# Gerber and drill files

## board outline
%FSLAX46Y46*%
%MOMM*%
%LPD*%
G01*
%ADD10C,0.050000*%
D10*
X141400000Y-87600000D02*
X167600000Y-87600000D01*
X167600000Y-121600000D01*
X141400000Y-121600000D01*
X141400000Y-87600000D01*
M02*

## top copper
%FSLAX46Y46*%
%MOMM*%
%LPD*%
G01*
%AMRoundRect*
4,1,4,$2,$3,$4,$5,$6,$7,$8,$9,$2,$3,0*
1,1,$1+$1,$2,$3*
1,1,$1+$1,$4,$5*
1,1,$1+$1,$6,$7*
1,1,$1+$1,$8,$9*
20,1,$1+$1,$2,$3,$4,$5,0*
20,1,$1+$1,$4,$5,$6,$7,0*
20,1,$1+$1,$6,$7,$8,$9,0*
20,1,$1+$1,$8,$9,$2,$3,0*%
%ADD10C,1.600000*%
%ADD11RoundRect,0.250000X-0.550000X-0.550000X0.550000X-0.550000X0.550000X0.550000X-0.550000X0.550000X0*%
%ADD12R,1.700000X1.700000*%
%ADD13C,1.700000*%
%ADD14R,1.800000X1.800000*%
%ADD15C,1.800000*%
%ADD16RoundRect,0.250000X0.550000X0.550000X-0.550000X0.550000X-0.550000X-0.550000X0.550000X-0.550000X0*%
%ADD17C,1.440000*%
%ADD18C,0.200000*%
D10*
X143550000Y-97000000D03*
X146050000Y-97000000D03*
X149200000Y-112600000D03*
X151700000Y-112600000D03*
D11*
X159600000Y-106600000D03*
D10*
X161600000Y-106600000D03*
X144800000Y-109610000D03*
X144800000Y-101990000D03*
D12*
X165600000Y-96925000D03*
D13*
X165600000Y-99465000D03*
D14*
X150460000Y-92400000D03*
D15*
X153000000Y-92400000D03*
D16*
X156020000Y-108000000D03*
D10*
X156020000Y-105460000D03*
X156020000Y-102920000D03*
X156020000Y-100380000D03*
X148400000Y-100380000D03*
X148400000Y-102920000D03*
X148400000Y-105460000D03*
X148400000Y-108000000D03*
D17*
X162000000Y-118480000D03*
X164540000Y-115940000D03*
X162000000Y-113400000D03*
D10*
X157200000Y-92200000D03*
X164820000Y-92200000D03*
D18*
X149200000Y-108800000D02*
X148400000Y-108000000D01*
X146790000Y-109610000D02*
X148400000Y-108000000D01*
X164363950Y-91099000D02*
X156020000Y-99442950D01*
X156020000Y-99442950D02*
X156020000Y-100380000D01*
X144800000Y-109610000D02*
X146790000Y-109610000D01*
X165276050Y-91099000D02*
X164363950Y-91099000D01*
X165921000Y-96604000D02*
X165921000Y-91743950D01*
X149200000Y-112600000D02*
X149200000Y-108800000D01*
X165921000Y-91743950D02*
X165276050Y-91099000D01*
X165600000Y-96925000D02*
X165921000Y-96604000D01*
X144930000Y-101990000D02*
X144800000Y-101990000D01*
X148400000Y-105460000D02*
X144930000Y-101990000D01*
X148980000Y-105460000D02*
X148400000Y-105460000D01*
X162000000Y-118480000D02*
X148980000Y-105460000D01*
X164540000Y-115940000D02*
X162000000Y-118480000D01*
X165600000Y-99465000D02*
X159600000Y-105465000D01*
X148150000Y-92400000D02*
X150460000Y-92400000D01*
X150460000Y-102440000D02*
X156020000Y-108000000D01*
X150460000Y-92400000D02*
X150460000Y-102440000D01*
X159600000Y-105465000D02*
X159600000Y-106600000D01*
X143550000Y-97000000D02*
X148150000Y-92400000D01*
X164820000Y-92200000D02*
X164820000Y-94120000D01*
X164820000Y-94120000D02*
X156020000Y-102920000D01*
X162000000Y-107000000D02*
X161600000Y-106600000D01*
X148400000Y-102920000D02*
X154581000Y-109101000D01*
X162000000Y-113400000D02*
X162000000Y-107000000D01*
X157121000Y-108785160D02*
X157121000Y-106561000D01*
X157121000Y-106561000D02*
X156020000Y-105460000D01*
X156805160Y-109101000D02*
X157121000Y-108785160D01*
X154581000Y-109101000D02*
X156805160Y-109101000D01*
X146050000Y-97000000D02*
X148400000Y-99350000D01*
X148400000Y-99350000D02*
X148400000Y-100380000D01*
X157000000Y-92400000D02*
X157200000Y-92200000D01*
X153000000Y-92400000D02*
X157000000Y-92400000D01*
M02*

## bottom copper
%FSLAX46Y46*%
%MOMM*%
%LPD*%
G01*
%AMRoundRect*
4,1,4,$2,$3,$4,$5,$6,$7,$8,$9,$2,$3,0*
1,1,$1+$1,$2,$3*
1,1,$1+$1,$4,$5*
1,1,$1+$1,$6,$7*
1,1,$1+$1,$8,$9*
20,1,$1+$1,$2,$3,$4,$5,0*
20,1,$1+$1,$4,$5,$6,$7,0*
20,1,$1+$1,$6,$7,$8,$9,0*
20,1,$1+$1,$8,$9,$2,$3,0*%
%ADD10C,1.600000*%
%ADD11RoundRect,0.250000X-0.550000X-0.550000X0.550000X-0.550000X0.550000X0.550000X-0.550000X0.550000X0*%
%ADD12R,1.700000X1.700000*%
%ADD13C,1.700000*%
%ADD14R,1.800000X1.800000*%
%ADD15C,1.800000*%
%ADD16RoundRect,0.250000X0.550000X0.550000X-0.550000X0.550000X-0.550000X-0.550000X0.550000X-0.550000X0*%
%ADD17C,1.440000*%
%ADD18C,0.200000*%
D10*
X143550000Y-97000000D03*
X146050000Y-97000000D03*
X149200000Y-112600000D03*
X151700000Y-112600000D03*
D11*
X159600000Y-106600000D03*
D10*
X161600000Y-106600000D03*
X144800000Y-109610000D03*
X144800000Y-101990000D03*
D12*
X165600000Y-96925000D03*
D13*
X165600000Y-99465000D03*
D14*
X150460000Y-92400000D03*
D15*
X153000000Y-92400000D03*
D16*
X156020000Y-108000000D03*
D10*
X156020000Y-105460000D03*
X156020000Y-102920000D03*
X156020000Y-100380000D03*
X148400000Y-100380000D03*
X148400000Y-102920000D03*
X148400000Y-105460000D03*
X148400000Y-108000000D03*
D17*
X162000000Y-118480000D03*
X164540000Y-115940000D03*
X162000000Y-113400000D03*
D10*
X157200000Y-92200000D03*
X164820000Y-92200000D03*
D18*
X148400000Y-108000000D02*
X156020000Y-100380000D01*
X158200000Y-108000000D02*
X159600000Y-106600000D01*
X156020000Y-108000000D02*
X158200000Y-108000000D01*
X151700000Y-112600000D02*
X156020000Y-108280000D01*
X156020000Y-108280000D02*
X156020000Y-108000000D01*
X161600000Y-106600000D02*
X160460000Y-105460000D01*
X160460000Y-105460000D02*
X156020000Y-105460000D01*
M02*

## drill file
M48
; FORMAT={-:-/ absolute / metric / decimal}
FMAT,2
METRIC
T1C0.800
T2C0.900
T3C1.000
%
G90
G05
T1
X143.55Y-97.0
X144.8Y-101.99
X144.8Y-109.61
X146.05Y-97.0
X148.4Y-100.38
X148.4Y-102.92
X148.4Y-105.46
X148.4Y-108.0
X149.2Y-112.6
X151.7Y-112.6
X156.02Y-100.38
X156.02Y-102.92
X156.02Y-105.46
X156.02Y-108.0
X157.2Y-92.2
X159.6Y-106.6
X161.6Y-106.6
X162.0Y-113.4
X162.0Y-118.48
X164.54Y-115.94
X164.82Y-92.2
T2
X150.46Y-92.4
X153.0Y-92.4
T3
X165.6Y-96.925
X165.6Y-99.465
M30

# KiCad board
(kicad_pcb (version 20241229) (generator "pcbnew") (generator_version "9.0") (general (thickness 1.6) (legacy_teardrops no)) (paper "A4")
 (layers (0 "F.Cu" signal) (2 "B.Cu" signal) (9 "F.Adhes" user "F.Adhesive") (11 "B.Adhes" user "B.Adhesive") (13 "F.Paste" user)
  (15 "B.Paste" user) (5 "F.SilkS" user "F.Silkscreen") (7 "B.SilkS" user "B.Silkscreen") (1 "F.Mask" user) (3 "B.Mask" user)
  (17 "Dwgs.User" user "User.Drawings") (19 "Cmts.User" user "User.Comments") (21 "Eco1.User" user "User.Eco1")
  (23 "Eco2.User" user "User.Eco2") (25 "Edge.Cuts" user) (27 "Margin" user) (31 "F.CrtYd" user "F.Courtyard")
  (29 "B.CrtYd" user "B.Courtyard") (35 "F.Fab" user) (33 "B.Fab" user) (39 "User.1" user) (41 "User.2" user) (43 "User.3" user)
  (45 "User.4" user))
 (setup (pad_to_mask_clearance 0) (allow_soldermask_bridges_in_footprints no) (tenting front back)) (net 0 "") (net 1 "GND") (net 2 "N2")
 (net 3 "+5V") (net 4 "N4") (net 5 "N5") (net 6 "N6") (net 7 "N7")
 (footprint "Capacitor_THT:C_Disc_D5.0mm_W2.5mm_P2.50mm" (layer "F.Cu") (at 143.55 97)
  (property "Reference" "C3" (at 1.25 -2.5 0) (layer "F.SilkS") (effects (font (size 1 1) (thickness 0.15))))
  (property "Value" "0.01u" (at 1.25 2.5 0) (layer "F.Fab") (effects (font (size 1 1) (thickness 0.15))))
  (pad "1" thru_hole circle (at 0 0) (size 1.6 1.6) (drill 0.8) (layers "*.Cu" "*.Mask") (remove_unused_layers no) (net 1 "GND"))
  (pad "2" thru_hole circle (at 2.5 0) (size 1.6 1.6) (drill 0.8) (layers "*.Cu" "*.Mask") (remove_unused_layers no) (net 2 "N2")))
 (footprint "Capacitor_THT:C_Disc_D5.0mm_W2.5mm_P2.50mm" (layer "F.Cu") (at 149.2 112.6)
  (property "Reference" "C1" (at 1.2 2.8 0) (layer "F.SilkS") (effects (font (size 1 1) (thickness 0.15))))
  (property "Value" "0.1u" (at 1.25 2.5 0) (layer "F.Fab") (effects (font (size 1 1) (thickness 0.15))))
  (pad "1" thru_hole circle (at 0 0) (size 1.6 1.6) (drill 0.8) (layers "*.Cu" "*.Mask") (remove_unused_layers no) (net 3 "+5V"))
  (pad "2" thru_hole circle (at 2.5 0) (size 1.6 1.6) (drill 0.8) (layers "*.Cu" "*.Mask") (remove_unused_layers no) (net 1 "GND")))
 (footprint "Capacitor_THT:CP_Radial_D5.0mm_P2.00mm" (layer "F.Cu") (at 159.6 106.6)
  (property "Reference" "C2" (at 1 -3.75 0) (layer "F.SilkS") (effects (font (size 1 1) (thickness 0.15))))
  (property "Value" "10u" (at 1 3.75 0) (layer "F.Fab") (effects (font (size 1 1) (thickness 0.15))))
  (pad "1" thru_hole roundrect (at 0 0) (size 1.6 1.6) (drill 0.8) (layers "*.Cu" "*.Mask") (remove_unused_layers no)
   (roundrect_rratio 0.15625) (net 1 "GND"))
  (pad "2" thru_hole circle (at 2 0) (size 1.6 1.6) (drill 0.8) (layers "*.Cu" "*.Mask") (remove_unused_layers no) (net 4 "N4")))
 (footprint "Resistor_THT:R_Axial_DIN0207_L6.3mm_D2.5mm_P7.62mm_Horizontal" (layer "F.Cu") (at 144.8 109.61 90)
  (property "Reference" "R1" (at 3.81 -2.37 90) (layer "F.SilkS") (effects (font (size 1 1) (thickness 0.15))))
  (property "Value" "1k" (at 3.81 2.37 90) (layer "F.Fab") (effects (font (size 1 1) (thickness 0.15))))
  (pad "1" thru_hole circle (at 0 0 90) (size 1.6 1.6) (drill 0.8) (layers "*.Cu" "*.Mask") (remove_unused_layers no) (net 3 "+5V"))
  (pad "2" thru_hole circle (at 7.62 0 90) (size 1.6 1.6) (drill 0.8) (layers "*.Cu" "*.Mask") (remove_unused_layers no) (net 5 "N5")))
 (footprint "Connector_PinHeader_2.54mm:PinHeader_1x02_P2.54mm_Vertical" (layer "F.Cu") (at 165.6 96.925)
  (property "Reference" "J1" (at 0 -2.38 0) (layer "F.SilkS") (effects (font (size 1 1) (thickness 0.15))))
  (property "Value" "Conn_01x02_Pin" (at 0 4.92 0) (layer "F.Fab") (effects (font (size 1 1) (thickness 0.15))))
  (pad "1" thru_hole rect (at 0 0) (size 1.7 1.7) (drill 1) (layers "*.Cu" "*.Mask") (remove_unused_layers no) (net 3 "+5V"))
  (pad "2" thru_hole circle (at 0 2.54) (size 1.7 1.7) (drill 1) (layers "*.Cu" "*.Mask") (remove_unused_layers no) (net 1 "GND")))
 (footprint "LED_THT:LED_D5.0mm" (layer "F.Cu") (at 150.46 92.4)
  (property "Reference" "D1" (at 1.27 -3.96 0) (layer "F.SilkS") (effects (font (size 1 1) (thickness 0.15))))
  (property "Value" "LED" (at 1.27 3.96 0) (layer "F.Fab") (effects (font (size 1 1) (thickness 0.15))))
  (pad "1" thru_hole rect (at 0 0) (size 1.8 1.8) (drill 0.9) (layers "*.Cu" "*.Mask") (remove_unused_layers no) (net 1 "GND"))
  (pad "2" thru_hole circle (at 2.54 0) (size 1.8 1.8) (drill 0.9) (layers "*.Cu" "*.Mask") (remove_unused_layers no) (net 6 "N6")))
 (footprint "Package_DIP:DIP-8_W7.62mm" (layer "F.Cu") (at 156.02 108 180)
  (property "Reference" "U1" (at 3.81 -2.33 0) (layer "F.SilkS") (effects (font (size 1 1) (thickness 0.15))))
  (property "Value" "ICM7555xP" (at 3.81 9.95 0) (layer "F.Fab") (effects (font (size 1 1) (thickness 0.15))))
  (pad "1" thru_hole roundrect (at 0 0 180) (size 1.6 1.6) (drill 0.8) (layers "*.Cu" "*.Mask") (remove_unused_layers no)
   (roundrect_rratio 0.15625) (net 1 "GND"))
  (pad "2" thru_hole circle (at 0 2.54 180) (size 1.6 1.6) (drill 0.8) (layers "*.Cu" "*.Mask") (remove_unused_layers no) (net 4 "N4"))
  (pad "3" thru_hole circle (at 0 5.08 180) (size 1.6 1.6) (drill 0.8) (layers "*.Cu" "*.Mask") (remove_unused_layers no) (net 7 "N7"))
  (pad "4" thru_hole circle (at 0 7.62 180) (size 1.6 1.6) (drill 0.8) (layers "*.Cu" "*.Mask") (remove_unused_layers no) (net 3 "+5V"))
  (pad "5" thru_hole circle (at 7.62 7.62 180) (size 1.6 1.6) (drill 0.8) (layers "*.Cu" "*.Mask") (remove_unused_layers no) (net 2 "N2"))
  (pad "6" thru_hole circle (at 7.62 5.08 180) (size 1.6 1.6) (drill 0.8) (layers "*.Cu" "*.Mask") (remove_unused_layers no) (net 4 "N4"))
  (pad "7" thru_hole circle (at 7.62 2.54 180) (size 1.6 1.6) (drill 0.8) (layers "*.Cu" "*.Mask") (remove_unused_layers no) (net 5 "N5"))
  (pad "8" thru_hole circle (at 7.62 0 180) (size 1.6 1.6) (drill 0.8) (layers "*.Cu" "*.Mask") (remove_unused_layers no) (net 3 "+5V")))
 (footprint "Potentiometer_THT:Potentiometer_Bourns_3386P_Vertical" (layer "F.Cu") (at 162 118.48)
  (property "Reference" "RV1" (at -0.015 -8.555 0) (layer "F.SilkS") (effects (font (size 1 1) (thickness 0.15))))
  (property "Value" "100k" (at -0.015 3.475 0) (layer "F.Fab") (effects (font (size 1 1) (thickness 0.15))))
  (pad "1" thru_hole circle (at 0 0) (size 1.44 1.44) (drill 0.8) (layers "*.Cu" "*.Mask") (remove_unused_layers no) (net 5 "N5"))
  (pad "2" thru_hole circle (at 2.54 -2.54) (size 1.44 1.44) (drill 0.8) (layers "*.Cu" "*.Mask") (remove_unused_layers no) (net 5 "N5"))
  (pad "3" thru_hole circle (at 0 -5.08) (size 1.44 1.44) (drill 0.8) (layers "*.Cu" "*.Mask") (remove_unused_layers no) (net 4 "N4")))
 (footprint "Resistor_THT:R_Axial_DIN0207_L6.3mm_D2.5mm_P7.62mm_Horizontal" (layer "F.Cu") (at 157.2 92.2)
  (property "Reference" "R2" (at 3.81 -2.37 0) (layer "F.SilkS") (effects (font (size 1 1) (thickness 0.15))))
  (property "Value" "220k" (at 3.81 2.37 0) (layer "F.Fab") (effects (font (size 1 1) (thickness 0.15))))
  (pad "1" thru_hole circle (at 0 0) (size 1.6 1.6) (drill 0.8) (layers "*.Cu" "*.Mask") (remove_unused_layers no) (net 6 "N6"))
  (pad "2" thru_hole circle (at 7.62 0) (size 1.6 1.6) (drill 0.8) (layers "*.Cu" "*.Mask") (remove_unused_layers no) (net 7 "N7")))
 (gr_rect (start 141.4 87.6) (end 167.6 121.6) (stroke (width 0.05) (type default)) (fill no) (layer "Edge.Cuts"))
 (segment (start 149.2 108.8) (end 148.4 108) (width 0.2) (layer "F.Cu") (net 3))
 (segment (start 146.79 109.61) (end 148.4 108) (width 0.2) (layer "F.Cu") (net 3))
 (segment (start 164.36395 91.099) (end 156.02 99.44295) (width 0.2) (layer "F.Cu") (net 3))
 (segment (start 156.02 99.44295) (end 156.02 100.38) (width 0.2) (layer "F.Cu") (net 3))
 (segment (start 144.8 109.61) (end 146.79 109.61) (width 0.2) (layer "F.Cu") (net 3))
 (segment (start 165.27605 91.099) (end 164.36395 91.099) (width 0.2) (layer "F.Cu") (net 3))
 (segment (start 165.921 96.604) (end 165.921 91.74395) (width 0.2) (layer "F.Cu") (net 3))
 (segment (start 149.2 112.6) (end 149.2 108.8) (width 0.2) (layer "F.Cu") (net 3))
 (segment (start 165.921 91.74395) (end 165.27605 91.099) (width 0.2) (layer "F.Cu") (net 3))
 (segment (start 165.6 96.925) (end 165.921 96.604) (width 0.2) (layer "F.Cu") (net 3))
 (segment (start 148.4 108) (end 156.02 100.38) (width 0.2) (layer "B.Cu") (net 3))
 (segment (start 144.93 101.99) (end 144.8 101.99) (width 0.2) (layer "F.Cu") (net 5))
 (segment (start 148.4 105.46) (end 144.93 101.99) (width 0.2) (layer "F.Cu") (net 5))
 (segment (start 148.98 105.46) (end 148.4 105.46) (width 0.2) (layer "F.Cu") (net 5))
 (segment (start 162 118.48) (end 148.98 105.46) (width 0.2) (layer "F.Cu") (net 5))
 (segment (start 164.54 115.94) (end 162 118.48) (width 0.2) (layer "F.Cu") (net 5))
 (segment (start 165.6 99.465) (end 159.6 105.465) (width 0.2) (layer "F.Cu") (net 1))
 (segment (start 148.15 92.4) (end 150.46 92.4) (width 0.2) (layer "F.Cu") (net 1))
 (segment (start 150.46 102.44) (end 156.02 108) (width 0.2) (layer "F.Cu") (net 1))
 (segment (start 150.46 92.4) (end 150.46 102.44) (width 0.2) (layer "F.Cu") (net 1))
 (segment (start 159.6 105.465) (end 159.6 106.6) (width 0.2) (layer "F.Cu") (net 1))
 (segment (start 143.55 97) (end 148.15 92.4) (width 0.2) (layer "F.Cu") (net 1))
 (segment (start 158.2 108) (end 159.6 106.6) (width 0.2) (layer "B.Cu") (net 1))
 (segment (start 156.02 108) (end 158.2 108) (width 0.2) (layer "B.Cu") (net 1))
 (segment (start 151.7 112.6) (end 156.02 108.28) (width 0.2) (layer "B.Cu") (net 1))
 (segment (start 156.02 108.28) (end 156.02 108) (width 0.2) (layer "B.Cu") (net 1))
 (segment (start 164.82 92.2) (end 164.82 94.12) (width 0.2) (layer "F.Cu") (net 7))
 (segment (start 164.82 94.12) (end 156.02 102.92) (width 0.2) (layer "F.Cu") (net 7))
 (segment (start 162 107) (end 161.6 106.6) (width 0.2) (layer "F.Cu") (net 4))
 (segment (start 148.4 102.92) (end 154.581 109.101) (width 0.2) (layer "F.Cu") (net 4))
 (segment (start 162 113.4) (end 162 107) (width 0.2) (layer "F.Cu") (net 4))
 (segment (start 157.121 108.78516) (end 157.121 106.561) (width 0.2) (layer "F.Cu") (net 4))
 (segment (start 157.121 106.561) (end 156.02 105.46) (width 0.2) (layer "F.Cu") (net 4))
 (segment (start 156.80516 109.101) (end 157.121 108.78516) (width 0.2) (layer "F.Cu") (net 4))
 (segment (start 154.581 109.101) (end 156.80516 109.101) (width 0.2) (layer "F.Cu") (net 4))
 (segment (start 161.6 106.6) (end 160.46 105.46) (width 0.2) (layer "B.Cu") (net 4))
 (segment (start 160.46 105.46) (end 156.02 105.46) (width 0.2) (layer "B.Cu") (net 4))
 (segment (start 146.05 97) (end 148.4 99.35) (width 0.2) (layer "F.Cu") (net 2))
 (segment (start 148.4 99.35) (end 148.4 100.38) (width 0.2) (layer "F.Cu") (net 2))
 (segment (start 157 92.4) (end 157.2 92.2) (width 0.2) (layer "F.Cu") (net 6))
 (segment (start 153 92.4) (end 157 92.4) (width 0.2) (layer "F.Cu") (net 6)))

